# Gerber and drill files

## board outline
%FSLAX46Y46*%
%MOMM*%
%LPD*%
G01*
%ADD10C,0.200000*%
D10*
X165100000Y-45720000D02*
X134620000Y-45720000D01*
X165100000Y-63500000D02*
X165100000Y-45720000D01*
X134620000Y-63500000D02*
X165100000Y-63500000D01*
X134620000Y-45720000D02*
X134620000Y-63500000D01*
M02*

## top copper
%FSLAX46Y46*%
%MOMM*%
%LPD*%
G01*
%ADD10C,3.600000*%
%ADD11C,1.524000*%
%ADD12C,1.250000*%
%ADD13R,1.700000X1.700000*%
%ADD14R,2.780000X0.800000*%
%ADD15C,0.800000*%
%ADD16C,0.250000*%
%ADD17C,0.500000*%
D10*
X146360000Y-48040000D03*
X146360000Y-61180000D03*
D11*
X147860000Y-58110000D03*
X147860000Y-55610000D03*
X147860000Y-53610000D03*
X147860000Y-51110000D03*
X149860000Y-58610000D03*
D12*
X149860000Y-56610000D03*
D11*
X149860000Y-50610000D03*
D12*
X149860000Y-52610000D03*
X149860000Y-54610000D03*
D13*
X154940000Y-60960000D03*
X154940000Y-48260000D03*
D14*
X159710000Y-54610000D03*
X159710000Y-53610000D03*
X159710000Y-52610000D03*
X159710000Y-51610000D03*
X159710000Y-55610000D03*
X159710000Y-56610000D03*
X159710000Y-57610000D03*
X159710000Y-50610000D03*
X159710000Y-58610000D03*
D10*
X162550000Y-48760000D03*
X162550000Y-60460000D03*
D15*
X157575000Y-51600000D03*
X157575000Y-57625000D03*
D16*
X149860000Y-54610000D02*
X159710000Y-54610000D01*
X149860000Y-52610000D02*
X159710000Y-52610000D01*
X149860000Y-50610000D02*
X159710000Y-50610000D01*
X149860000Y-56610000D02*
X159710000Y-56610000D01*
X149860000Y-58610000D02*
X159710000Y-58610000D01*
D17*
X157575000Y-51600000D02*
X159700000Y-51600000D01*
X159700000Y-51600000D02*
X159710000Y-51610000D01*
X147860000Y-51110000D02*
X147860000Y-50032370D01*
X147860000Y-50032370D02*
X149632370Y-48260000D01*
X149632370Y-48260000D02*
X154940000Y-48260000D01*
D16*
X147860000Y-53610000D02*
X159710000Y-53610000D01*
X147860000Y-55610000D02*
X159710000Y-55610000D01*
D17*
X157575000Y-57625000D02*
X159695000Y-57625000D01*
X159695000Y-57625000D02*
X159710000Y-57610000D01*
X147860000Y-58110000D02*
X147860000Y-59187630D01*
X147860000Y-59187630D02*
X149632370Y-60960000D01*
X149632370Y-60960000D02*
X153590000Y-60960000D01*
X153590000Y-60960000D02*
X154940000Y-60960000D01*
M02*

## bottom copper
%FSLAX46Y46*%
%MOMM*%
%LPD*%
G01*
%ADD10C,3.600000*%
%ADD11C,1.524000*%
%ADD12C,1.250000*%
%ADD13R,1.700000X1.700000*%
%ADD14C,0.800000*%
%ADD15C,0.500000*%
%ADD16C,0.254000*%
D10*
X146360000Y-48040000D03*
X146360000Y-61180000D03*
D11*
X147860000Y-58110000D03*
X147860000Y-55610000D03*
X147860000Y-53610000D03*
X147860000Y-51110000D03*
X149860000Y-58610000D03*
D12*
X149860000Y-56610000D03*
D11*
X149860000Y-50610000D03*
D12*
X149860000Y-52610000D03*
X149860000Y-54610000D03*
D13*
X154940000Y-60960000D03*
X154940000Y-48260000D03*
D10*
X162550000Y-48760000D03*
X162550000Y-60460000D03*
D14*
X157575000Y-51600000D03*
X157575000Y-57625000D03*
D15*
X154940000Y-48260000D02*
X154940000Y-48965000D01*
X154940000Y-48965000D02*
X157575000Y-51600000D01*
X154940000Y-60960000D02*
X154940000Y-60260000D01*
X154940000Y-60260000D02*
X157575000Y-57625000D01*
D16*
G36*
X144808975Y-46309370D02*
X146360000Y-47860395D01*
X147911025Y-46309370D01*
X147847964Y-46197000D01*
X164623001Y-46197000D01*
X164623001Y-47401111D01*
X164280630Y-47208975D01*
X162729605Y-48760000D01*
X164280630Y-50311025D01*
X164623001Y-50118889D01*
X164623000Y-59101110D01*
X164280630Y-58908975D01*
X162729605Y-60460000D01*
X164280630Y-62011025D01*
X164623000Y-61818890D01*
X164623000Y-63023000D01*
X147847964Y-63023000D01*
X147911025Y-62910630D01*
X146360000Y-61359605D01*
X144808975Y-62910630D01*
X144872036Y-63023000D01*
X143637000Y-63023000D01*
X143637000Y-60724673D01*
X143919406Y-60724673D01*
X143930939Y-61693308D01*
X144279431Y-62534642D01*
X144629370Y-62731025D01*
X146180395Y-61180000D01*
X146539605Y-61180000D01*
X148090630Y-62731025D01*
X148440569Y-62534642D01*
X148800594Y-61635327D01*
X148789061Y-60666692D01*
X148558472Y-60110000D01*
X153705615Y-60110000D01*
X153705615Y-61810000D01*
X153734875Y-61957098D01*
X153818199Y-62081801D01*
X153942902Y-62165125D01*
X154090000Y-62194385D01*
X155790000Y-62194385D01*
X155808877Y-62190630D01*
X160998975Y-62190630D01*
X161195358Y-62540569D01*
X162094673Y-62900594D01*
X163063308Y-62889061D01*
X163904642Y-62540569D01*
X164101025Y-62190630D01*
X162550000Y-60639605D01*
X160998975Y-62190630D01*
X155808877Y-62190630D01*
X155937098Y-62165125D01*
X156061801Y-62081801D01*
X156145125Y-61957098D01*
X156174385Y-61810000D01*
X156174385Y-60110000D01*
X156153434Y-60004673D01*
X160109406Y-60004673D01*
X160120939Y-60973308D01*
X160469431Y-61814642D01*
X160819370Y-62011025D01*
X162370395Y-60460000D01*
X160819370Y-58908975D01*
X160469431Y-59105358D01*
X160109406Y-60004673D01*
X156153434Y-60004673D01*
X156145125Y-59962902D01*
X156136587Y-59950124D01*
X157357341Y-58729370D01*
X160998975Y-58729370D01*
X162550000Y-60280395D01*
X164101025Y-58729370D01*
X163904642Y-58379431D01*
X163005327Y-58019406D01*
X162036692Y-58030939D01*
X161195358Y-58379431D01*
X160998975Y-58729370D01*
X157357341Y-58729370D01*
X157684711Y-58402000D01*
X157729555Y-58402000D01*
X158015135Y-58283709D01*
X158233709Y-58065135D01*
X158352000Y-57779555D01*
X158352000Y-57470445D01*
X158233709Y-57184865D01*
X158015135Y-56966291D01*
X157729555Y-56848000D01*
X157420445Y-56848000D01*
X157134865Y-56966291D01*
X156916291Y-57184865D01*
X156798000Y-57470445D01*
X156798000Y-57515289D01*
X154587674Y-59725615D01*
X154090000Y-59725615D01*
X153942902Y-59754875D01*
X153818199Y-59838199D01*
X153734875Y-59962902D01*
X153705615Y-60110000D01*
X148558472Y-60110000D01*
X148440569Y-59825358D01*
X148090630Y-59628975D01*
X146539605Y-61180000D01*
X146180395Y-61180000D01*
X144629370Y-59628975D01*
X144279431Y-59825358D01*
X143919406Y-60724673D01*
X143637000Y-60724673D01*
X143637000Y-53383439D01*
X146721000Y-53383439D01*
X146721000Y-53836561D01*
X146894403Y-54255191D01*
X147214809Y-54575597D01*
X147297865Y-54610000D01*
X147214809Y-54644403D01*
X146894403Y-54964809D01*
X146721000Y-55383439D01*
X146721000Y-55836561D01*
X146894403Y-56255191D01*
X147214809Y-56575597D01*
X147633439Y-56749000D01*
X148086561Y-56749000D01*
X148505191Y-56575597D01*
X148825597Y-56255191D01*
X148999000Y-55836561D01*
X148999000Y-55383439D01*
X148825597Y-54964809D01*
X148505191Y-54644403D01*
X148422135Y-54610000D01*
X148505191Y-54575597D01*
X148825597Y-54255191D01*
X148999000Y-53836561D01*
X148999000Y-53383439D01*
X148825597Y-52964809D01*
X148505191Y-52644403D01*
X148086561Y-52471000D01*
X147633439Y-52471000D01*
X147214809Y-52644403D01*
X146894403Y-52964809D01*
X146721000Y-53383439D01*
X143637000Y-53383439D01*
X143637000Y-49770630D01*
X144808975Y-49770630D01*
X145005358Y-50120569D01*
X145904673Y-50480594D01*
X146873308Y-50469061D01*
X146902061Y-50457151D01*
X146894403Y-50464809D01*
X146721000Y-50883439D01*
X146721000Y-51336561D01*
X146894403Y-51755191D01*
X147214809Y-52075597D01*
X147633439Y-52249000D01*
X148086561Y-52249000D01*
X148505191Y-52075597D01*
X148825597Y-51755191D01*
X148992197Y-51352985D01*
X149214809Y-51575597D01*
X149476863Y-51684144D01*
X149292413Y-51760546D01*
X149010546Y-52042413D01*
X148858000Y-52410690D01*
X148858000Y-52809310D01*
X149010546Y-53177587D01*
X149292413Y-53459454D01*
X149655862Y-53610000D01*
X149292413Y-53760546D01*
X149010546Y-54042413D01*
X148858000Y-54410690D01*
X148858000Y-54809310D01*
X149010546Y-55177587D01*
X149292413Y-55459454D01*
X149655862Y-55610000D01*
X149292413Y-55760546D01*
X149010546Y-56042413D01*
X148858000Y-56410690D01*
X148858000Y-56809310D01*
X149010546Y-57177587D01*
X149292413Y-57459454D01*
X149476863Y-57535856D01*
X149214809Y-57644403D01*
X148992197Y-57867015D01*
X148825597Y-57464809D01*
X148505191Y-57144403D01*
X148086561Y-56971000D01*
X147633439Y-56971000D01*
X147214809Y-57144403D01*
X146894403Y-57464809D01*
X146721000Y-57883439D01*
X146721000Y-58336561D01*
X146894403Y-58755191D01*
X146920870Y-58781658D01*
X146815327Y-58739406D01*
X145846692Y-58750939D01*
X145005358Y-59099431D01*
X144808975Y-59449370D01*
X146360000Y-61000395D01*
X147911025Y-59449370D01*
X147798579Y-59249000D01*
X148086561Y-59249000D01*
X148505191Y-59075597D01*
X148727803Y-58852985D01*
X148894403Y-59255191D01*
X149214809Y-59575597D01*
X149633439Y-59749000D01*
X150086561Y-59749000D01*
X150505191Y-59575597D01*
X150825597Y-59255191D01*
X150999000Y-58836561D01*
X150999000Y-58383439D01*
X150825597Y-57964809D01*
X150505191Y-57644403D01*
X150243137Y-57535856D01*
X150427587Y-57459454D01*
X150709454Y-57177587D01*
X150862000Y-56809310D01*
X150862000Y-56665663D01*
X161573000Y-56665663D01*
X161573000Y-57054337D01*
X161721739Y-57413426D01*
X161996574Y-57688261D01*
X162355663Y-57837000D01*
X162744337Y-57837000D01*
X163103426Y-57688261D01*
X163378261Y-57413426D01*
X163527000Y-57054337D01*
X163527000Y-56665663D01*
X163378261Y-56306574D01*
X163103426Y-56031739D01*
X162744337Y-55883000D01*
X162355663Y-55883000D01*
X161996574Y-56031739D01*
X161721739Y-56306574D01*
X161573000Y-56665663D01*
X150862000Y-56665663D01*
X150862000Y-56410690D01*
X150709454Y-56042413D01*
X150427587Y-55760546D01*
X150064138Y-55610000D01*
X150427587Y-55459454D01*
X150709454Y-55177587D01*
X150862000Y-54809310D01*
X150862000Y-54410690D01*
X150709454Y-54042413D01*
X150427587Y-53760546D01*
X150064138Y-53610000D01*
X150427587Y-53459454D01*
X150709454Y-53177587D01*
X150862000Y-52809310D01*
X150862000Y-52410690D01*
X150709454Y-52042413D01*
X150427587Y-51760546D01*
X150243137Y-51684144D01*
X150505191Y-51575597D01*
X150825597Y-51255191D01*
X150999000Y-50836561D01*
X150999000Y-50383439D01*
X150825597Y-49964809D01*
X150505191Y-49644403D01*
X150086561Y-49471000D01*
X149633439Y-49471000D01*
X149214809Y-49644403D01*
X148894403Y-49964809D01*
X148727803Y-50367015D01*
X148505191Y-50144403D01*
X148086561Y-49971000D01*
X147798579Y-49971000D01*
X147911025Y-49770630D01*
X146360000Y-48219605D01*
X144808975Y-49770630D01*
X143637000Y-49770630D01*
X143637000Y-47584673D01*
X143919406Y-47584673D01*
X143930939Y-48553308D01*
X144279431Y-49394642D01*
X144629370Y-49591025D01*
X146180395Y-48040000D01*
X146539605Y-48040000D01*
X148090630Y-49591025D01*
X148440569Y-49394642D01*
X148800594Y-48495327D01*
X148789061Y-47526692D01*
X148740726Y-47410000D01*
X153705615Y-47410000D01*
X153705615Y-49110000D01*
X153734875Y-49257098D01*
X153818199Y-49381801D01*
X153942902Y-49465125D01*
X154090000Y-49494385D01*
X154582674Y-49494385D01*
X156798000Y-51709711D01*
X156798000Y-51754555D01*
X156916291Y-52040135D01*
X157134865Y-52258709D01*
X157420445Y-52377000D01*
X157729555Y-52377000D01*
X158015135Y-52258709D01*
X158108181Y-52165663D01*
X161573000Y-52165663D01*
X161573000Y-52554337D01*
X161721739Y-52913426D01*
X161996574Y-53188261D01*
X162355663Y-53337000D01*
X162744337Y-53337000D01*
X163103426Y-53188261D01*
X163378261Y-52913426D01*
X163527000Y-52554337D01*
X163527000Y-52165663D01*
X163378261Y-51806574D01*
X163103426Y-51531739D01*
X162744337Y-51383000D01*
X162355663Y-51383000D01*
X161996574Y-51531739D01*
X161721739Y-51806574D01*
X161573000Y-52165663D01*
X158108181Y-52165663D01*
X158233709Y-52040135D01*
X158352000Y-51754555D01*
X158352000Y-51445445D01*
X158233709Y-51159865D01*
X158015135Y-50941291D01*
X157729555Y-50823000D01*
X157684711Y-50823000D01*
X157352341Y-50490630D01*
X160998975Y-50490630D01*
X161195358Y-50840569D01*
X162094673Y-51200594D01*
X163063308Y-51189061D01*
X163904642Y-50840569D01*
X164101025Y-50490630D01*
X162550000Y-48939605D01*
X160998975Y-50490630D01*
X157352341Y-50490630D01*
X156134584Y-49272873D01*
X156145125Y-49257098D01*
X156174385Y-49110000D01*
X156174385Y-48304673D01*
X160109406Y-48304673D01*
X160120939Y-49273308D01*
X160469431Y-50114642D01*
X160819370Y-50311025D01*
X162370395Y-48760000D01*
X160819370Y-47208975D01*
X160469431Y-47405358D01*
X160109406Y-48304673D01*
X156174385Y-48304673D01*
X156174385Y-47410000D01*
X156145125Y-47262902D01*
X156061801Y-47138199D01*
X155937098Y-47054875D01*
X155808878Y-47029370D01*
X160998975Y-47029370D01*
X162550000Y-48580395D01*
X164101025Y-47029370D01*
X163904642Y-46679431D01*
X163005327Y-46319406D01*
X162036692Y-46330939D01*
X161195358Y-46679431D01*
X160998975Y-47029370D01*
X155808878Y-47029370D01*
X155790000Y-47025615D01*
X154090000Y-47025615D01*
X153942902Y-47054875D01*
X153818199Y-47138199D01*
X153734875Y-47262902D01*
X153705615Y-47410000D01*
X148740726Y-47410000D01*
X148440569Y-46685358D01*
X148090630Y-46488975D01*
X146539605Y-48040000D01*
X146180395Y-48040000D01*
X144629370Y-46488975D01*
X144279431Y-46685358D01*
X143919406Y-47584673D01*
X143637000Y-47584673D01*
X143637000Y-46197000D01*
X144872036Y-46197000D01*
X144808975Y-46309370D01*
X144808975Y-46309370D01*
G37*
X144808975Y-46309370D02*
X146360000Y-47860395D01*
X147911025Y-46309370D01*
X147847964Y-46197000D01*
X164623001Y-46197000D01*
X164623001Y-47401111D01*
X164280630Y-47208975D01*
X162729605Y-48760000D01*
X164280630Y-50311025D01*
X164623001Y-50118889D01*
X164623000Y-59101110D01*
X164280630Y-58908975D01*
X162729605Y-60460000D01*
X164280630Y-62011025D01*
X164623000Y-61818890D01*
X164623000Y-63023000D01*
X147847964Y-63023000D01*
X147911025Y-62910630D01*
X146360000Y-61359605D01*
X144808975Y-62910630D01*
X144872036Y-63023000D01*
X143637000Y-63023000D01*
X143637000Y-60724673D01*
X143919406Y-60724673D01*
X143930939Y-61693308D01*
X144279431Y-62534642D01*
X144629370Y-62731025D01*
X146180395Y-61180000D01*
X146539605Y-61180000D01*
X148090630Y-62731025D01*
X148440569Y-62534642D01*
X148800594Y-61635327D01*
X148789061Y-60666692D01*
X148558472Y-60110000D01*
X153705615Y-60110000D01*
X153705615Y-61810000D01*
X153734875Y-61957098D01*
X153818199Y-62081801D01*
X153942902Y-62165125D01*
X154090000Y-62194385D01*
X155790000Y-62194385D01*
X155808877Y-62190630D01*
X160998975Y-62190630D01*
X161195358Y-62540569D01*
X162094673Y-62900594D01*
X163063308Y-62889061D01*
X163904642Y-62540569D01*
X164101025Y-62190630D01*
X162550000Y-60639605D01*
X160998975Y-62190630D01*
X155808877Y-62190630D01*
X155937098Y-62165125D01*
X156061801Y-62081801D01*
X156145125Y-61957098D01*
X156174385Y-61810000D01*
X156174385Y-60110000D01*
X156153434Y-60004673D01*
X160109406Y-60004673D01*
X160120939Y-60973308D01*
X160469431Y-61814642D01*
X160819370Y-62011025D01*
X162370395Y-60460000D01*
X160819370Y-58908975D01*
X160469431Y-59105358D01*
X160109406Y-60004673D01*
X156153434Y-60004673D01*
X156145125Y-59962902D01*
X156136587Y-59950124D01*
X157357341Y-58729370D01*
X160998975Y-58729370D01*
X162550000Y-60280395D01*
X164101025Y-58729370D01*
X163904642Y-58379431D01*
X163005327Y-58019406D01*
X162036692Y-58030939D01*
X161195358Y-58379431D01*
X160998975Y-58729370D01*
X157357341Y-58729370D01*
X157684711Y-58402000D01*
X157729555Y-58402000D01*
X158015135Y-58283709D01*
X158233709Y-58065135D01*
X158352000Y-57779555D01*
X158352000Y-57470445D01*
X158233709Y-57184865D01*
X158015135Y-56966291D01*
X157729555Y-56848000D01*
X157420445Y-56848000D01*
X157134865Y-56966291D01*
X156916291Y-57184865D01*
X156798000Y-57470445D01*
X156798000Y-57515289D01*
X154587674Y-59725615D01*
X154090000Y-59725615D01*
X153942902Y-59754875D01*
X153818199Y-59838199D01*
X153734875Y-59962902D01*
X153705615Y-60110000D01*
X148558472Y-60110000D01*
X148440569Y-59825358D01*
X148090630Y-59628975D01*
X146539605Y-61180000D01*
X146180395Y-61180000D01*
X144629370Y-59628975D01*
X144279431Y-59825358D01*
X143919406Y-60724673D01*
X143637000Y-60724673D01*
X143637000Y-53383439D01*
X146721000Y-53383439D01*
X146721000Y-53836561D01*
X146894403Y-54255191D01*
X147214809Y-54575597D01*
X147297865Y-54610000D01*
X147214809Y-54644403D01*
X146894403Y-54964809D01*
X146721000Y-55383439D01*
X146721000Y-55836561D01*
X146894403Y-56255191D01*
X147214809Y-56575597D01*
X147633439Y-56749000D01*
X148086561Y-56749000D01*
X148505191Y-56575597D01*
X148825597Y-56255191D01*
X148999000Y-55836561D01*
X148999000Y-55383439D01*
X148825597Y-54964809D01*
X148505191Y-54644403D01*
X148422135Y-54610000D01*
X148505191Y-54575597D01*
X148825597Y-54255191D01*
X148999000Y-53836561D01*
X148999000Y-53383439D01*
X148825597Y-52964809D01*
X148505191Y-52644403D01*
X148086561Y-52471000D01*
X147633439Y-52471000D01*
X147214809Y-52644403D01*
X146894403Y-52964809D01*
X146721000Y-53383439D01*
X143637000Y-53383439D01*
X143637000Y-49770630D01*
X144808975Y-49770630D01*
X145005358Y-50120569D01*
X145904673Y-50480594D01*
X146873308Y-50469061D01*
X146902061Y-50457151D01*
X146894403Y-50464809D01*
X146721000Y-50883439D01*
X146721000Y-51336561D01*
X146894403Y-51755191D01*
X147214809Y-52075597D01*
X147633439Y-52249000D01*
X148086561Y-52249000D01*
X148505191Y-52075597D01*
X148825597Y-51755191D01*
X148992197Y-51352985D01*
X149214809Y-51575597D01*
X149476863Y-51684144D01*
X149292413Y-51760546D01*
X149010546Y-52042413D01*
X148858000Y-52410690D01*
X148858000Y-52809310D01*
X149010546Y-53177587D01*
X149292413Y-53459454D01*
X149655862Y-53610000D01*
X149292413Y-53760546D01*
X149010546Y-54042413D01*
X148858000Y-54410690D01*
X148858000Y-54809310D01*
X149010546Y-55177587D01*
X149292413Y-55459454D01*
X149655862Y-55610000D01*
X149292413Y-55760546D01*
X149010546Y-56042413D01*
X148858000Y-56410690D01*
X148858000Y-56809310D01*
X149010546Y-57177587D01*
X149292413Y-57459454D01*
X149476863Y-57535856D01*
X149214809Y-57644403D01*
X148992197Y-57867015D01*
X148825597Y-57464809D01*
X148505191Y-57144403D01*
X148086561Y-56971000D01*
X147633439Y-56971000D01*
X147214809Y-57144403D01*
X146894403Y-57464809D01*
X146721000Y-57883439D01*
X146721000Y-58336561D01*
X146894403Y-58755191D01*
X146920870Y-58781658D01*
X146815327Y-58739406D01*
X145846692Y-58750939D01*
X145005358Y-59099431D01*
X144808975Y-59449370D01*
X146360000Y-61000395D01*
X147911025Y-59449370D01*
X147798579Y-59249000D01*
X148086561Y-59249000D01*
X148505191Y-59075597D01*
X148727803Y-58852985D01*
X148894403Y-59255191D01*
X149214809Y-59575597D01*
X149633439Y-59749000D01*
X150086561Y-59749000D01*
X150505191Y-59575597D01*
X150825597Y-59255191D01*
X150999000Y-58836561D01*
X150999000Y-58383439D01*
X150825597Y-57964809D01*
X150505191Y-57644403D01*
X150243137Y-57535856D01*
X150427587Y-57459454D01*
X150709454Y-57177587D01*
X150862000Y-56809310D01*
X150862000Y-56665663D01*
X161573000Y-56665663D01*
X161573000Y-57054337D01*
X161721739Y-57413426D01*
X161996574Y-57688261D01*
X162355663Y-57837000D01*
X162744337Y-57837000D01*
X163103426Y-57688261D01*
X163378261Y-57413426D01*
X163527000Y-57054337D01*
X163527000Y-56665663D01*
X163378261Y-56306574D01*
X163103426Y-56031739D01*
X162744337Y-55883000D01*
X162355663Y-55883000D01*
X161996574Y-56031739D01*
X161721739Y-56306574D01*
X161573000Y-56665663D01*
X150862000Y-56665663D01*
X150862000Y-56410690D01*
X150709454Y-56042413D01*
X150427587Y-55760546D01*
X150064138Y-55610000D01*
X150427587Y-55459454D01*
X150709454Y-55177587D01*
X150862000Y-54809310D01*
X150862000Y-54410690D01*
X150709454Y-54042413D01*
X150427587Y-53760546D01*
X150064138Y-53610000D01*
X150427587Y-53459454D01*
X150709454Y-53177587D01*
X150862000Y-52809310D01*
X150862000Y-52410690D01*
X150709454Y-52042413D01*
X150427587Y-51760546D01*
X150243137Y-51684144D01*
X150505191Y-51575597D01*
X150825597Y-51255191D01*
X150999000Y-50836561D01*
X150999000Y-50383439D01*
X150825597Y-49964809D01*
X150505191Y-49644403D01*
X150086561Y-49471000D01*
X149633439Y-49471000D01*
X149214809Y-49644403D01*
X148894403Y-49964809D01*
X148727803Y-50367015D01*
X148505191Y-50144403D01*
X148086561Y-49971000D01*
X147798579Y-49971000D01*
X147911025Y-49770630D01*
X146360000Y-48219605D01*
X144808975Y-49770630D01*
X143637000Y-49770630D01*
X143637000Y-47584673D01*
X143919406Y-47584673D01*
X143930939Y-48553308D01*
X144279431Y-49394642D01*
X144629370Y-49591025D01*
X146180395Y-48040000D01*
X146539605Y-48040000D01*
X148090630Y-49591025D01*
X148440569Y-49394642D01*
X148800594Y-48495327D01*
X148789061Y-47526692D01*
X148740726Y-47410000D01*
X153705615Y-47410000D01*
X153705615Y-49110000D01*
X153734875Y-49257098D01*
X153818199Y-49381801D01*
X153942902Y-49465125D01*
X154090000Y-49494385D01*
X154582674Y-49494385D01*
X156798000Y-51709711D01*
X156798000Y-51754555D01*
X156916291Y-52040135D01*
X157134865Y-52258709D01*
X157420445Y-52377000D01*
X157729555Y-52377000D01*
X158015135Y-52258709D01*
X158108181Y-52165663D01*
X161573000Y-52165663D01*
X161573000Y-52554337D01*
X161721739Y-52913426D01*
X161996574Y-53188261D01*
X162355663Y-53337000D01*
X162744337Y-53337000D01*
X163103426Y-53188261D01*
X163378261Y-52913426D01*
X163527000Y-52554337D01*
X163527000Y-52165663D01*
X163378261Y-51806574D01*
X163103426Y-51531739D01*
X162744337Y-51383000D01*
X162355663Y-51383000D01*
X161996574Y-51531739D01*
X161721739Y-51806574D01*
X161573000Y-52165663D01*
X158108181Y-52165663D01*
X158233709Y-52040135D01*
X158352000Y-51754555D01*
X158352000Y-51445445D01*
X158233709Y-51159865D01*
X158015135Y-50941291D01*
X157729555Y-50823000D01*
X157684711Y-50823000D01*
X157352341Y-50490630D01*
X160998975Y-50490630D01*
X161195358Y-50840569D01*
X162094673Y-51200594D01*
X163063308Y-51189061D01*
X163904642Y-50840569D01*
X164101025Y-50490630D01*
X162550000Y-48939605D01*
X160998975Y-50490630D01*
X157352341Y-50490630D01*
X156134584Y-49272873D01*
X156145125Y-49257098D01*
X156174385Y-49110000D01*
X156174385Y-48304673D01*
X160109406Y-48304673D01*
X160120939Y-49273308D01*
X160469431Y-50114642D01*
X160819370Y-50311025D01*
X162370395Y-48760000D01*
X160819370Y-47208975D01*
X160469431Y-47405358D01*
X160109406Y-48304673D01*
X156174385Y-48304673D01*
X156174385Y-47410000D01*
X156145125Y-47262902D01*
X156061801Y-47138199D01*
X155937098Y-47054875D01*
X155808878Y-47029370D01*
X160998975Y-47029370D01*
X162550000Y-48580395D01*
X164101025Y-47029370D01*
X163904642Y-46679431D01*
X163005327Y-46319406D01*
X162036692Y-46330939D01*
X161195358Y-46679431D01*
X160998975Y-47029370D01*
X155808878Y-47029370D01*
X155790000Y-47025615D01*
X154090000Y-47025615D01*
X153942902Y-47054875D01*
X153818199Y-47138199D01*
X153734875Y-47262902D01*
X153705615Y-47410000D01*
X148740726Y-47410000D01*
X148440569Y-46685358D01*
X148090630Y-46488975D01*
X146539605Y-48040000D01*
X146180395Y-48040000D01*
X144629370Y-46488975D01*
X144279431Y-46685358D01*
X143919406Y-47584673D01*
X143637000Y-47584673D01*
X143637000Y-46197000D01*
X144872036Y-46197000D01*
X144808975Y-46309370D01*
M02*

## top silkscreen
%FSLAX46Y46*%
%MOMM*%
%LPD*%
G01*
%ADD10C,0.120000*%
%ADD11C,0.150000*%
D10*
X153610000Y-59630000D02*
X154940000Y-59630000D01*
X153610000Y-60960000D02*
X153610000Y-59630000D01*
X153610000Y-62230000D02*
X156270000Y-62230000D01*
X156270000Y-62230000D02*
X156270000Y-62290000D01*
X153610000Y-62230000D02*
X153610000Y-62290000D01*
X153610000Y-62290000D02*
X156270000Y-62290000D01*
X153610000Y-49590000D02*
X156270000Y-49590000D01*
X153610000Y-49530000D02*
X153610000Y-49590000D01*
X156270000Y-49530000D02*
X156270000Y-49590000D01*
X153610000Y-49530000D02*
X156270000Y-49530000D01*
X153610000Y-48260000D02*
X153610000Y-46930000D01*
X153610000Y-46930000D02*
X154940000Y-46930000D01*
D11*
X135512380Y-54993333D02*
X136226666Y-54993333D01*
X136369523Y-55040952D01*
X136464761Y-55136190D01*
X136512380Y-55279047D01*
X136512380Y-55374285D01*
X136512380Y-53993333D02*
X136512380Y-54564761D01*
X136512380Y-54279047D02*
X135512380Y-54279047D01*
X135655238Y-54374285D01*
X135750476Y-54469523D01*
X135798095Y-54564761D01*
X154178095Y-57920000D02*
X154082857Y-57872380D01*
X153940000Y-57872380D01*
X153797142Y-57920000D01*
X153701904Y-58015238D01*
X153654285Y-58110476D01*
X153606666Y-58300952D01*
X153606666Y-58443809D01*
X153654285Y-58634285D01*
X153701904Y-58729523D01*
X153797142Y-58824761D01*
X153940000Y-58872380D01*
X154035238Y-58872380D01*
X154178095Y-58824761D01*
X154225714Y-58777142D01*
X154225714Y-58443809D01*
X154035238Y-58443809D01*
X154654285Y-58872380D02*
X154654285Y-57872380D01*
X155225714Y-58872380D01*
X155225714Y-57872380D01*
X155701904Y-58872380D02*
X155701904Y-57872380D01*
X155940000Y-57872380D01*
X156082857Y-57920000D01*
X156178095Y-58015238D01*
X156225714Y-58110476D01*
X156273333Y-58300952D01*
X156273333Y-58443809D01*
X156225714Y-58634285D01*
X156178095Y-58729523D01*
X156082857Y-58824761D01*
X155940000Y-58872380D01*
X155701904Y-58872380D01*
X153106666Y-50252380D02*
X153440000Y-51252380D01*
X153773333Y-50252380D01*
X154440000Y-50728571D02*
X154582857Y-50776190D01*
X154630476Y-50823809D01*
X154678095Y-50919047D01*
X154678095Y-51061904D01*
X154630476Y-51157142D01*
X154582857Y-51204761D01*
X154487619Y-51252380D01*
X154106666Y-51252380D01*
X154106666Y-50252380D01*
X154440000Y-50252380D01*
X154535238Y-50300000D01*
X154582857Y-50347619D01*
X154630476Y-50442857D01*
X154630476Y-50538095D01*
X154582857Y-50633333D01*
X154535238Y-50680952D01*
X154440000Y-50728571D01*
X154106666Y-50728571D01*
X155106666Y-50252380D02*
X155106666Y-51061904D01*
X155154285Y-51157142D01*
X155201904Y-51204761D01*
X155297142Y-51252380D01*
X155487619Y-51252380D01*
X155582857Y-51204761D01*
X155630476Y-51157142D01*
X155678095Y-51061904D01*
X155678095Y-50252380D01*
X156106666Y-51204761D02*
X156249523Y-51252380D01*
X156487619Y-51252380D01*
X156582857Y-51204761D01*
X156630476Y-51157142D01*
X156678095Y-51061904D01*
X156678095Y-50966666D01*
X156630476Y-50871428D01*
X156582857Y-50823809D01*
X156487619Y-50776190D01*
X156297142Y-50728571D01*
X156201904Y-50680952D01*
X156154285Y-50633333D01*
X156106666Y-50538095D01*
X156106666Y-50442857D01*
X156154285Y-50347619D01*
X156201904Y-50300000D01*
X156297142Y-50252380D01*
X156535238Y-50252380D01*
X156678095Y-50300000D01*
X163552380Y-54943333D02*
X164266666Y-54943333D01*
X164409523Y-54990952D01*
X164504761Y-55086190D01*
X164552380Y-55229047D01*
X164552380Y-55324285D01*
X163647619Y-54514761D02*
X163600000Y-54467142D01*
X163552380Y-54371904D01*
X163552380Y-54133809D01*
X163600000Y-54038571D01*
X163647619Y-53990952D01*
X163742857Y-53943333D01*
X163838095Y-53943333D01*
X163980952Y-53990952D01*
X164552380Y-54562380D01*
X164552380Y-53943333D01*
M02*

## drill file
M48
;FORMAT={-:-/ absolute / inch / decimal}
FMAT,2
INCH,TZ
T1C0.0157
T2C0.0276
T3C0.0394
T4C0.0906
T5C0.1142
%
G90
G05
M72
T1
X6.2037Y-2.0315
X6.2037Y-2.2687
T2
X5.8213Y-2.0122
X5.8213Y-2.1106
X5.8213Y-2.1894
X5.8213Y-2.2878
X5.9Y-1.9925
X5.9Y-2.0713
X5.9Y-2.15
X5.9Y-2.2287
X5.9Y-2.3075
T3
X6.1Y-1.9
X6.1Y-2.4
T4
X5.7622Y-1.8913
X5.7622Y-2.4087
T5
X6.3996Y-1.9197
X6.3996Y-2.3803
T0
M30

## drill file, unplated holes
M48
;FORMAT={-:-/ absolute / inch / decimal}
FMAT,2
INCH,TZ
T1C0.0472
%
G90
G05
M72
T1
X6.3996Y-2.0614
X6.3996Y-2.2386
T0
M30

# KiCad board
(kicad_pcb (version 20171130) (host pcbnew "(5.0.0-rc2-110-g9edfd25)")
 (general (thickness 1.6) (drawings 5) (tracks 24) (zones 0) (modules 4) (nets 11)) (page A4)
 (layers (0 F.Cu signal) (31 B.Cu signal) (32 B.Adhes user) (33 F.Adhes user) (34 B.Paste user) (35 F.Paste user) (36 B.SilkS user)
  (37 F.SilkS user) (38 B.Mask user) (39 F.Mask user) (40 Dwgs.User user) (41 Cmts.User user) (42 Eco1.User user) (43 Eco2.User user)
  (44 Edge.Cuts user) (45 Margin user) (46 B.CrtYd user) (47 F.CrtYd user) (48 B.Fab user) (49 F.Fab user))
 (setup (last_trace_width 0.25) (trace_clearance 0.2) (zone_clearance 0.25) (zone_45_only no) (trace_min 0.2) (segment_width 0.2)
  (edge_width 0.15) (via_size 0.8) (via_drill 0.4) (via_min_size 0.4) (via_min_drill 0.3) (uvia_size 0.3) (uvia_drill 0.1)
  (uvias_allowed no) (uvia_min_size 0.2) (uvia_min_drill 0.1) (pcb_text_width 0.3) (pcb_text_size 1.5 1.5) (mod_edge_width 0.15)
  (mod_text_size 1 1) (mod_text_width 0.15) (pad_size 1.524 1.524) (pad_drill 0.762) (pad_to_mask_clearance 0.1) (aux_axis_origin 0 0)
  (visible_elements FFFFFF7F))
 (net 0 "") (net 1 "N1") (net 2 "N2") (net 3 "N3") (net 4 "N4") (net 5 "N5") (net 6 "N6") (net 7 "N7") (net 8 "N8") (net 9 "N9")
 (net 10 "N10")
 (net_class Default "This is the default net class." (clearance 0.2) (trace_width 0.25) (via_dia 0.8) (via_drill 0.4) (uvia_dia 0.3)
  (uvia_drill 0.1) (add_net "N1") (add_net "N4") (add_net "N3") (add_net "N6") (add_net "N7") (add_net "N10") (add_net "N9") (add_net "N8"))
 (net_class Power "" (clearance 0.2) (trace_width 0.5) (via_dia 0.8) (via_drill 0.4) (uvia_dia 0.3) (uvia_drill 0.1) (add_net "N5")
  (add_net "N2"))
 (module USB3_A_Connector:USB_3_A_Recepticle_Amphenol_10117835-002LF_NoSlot (layer F.Cu) (at 143.01 54.61 270)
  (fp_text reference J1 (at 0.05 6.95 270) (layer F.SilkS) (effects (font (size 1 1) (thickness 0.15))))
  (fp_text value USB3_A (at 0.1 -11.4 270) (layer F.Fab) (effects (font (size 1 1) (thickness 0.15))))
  (pad 10 thru_hole circle (at -6.57 -3.35 270) (size 3.6 3.6) (drill 2.3) (layers *.Cu *.Mask) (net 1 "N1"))
  (pad 10 thru_hole circle (at 6.57 -3.35 270) (size 3.6 3.6) (drill 2.3) (layers *.Cu *.Mask) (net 1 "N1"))
  (pad 4 thru_hole circle (at 3.5 -4.85 270) (size 1.524 1.524) (drill 0.7) (layers *.Cu *.Mask) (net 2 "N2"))
  (pad 3 thru_hole circle (at 1 -4.85 270) (size 1.524 1.524) (drill 0.7) (layers *.Cu *.Mask) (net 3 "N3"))
  (pad 2 thru_hole circle (at -1 -4.85 270) (size 1.524 1.524) (drill 0.7) (layers *.Cu *.Mask) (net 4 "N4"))
  (pad 1 thru_hole circle (at -3.5 -4.85 270) (size 1.524 1.524) (drill 0.7) (layers *.Cu *.Mask) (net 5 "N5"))
  (pad 5 thru_hole circle (at 4 -6.85 270) (size 1.524 1.524) (drill 0.7) (layers *.Cu *.Mask) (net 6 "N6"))
  (pad 6 thru_hole circle (at 2 -6.85 270) (size 1.25 1.25) (drill 0.7) (layers *.Cu *.Mask) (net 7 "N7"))
  (pad 9 thru_hole circle (at -4 -6.85 270) (size 1.524 1.524) (drill 0.7) (layers *.Cu *.Mask) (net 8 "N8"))
  (pad 8 thru_hole circle (at -2 -6.85 270) (size 1.25 1.25) (drill 0.7) (layers *.Cu *.Mask) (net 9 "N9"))
  (pad 7 thru_hole circle (at 0 -6.85 270) (size 1.25 1.25) (drill 0.7) (layers *.Cu *.Mask) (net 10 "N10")))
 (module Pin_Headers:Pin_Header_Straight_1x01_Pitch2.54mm (layer F.Cu) (at 154.94 60.96)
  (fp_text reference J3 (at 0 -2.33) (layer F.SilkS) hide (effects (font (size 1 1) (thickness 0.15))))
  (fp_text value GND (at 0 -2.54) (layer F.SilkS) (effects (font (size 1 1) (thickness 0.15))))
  (fp_line (start -1.33 -1.33) (end 0 -1.33) (layer F.SilkS) (width 0.12))
  (fp_line (start -1.33 0) (end -1.33 -1.33) (layer F.SilkS) (width 0.12))
  (fp_line (start -1.33 1.27) (end 1.33 1.27) (layer F.SilkS) (width 0.12))
  (fp_line (start 1.33 1.27) (end 1.33 1.33) (layer F.SilkS) (width 0.12))
  (fp_line (start -1.33 1.27) (end -1.33 1.33) (layer F.SilkS) (width 0.12))
  (fp_line (start -1.33 1.33) (end 1.33 1.33) (layer F.SilkS) (width 0.12))
  (pad 1 thru_hole rect (at 0 0) (size 1.7 1.7) (drill 1) (layers *.Cu *.Mask) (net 2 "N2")))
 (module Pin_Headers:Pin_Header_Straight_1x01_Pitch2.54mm (layer F.Cu) (at 154.94 48.26)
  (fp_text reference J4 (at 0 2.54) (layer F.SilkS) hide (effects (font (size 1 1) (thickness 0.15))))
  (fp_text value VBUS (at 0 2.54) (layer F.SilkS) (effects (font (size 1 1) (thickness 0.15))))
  (fp_line (start -1.33 1.33) (end 1.33 1.33) (layer F.SilkS) (width 0.12))
  (fp_line (start -1.33 1.27) (end -1.33 1.33) (layer F.SilkS) (width 0.12))
  (fp_line (start 1.33 1.27) (end 1.33 1.33) (layer F.SilkS) (width 0.12))
  (fp_line (start -1.33 1.27) (end 1.33 1.27) (layer F.SilkS) (width 0.12))
  (fp_line (start -1.33 0) (end -1.33 -1.33) (layer F.SilkS) (width 0.12))
  (fp_line (start -1.33 -1.33) (end 0 -1.33) (layer F.SilkS) (width 0.12))
  (pad 1 thru_hole rect (at 0 0) (size 1.7 1.7) (drill 1) (layers *.Cu *.Mask) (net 5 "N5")))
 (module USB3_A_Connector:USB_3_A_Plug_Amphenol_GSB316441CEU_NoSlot (layer F.Cu) (at 165.1 54.61 90)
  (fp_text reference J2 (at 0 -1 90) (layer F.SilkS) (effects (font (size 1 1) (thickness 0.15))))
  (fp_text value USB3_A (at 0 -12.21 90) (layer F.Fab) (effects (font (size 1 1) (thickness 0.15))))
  (pad 7 smd rect (at 0 -5.39 90) (size 0.8 2.78) (layers F.Cu F.Paste F.Mask) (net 10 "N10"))
  (pad 2 smd rect (at 1 -5.39 90) (size 0.8 2.78) (layers F.Cu F.Paste F.Mask) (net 4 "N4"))
  (pad 8 smd rect (at 2 -5.39 90) (size 0.8 2.78) (layers F.Cu F.Paste F.Mask) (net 9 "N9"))
  (pad 1 smd rect (at 3 -5.39 90) (size 0.8 2.78) (layers F.Cu F.Paste F.Mask) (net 5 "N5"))
  (pad 3 smd rect (at -1 -5.39 90) (size 0.8 2.78) (layers F.Cu F.Paste F.Mask) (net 3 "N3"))
  (pad 6 smd rect (at -2 -5.39 90) (size 0.8 2.78) (layers F.Cu F.Paste F.Mask) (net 7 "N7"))
  (pad 4 smd rect (at -3 -5.39 90) (size 0.8 2.78) (layers F.Cu F.Paste F.Mask) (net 2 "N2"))
  (pad 9 smd rect (at 4 -5.39 90) (size 0.8 2.78) (layers F.Cu F.Paste F.Mask) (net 8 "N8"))
  (pad 5 smd rect (at -4 -5.39 90) (size 0.8 2.78) (layers F.Cu F.Paste F.Mask) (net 6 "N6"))
  (pad 10 thru_hole circle (at 5.85 -2.55 90) (size 3.6 3.6) (drill 2.9) (layers *.Cu *.Mask) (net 1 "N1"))
  (pad 10 thru_hole circle (at -5.85 -2.55 90) (size 3.6 3.6) (drill 2.9) (layers *.Cu *.Mask) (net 1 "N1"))
  (pad "" np_thru_hole circle (at 2.25 -2.55 90) (size 1.2 1.2) (drill 1.2) (layers *.Cu *.Mask))
  (pad "" np_thru_hole circle (at -2.25 -2.55 90) (size 1.2 1.2) (drill 1.2) (layers *.Cu *.Mask)))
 (gr_line (start 165.1 45.72) (end 134.62 45.72) (layer Edge.Cuts) (width 0.2))
 (gr_line (start 165.1 63.5) (end 165.1 45.72) (layer Edge.Cuts) (width 0.2))
 (gr_line (start 134.62 63.5) (end 165.1 63.5) (layer Edge.Cuts) (width 0.2))
 (gr_line (start 134.62 45.72) (end 134.62 63.5) (layer Edge.Cuts) (width 0.2))
 (segment (start 149.86 54.61) (end 159.71 54.61) (width 0.25) (layer F.Cu) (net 10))
 (segment (start 149.86 52.61) (end 159.71 52.61) (width 0.25) (layer F.Cu) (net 9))
 (segment (start 149.86 50.61) (end 159.71 50.61) (width 0.25) (layer F.Cu) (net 8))
 (segment (start 149.86 56.61) (end 159.71 56.61) (width 0.25) (layer F.Cu) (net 7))
 (segment (start 149.86 58.61) (end 159.71 58.61) (width 0.25) (layer F.Cu) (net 6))
 (segment (start 157.575 51.6) (end 159.7 51.6) (width 0.5) (layer F.Cu) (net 5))
 (segment (start 159.7 51.6) (end 159.71 51.61) (width 0.5) (layer F.Cu) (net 5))
 (segment (start 154.94 48.26) (end 154.94 48.965) (width 0.5) (layer B.Cu) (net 5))
 (segment (start 154.94 48.965) (end 157.575 51.6) (width 0.5) (layer B.Cu) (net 5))
 (via (at 157.575 51.6) (size 0.8) (drill 0.4) (layers F.Cu B.Cu) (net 5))
 (segment (start 147.86 51.11) (end 147.86 50.03237) (width 0.5) (layer F.Cu) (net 5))
 (segment (start 147.86 50.03237) (end 149.63237 48.26) (width 0.5) (layer F.Cu) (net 5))
 (segment (start 149.63237 48.26) (end 154.94 48.26) (width 0.5) (layer F.Cu) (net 5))
 (segment (start 147.86 53.61) (end 159.71 53.61) (width 0.25) (layer F.Cu) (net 4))
 (segment (start 147.86 55.61) (end 159.71 55.61) (width 0.25) (layer F.Cu) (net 3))
 (segment (start 157.575 57.625) (end 159.695 57.625) (width 0.5) (layer F.Cu) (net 2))
 (segment (start 159.695 57.625) (end 159.71 57.61) (width 0.5) (layer F.Cu) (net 2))
 (segment (start 154.94 60.96) (end 154.94 60.26) (width 0.5) (layer B.Cu) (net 2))
 (segment (start 154.94 60.26) (end 157.575 57.625) (width 0.5) (layer B.Cu) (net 2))
 (via (at 157.575 57.625) (size 0.8) (drill 0.4) (layers F.Cu B.Cu) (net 2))
 (segment (start 147.86 58.11) (end 147.86 59.18763) (width 0.5) (layer F.Cu) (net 2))
 (segment (start 147.86 59.18763) (end 149.63237 60.96) (width 0.5) (layer F.Cu) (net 2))
 (segment (start 149.63237 60.96) (end 153.59 60.96) (width 0.5) (layer F.Cu) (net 2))
 (segment (start 153.59 60.96) (end 154.94 60.96) (width 0.5) (layer F.Cu) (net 2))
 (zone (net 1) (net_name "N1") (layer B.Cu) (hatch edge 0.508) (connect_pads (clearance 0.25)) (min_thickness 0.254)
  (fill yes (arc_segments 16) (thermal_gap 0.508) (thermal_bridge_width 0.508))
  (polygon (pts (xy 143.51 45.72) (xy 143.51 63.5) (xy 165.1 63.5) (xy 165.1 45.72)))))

